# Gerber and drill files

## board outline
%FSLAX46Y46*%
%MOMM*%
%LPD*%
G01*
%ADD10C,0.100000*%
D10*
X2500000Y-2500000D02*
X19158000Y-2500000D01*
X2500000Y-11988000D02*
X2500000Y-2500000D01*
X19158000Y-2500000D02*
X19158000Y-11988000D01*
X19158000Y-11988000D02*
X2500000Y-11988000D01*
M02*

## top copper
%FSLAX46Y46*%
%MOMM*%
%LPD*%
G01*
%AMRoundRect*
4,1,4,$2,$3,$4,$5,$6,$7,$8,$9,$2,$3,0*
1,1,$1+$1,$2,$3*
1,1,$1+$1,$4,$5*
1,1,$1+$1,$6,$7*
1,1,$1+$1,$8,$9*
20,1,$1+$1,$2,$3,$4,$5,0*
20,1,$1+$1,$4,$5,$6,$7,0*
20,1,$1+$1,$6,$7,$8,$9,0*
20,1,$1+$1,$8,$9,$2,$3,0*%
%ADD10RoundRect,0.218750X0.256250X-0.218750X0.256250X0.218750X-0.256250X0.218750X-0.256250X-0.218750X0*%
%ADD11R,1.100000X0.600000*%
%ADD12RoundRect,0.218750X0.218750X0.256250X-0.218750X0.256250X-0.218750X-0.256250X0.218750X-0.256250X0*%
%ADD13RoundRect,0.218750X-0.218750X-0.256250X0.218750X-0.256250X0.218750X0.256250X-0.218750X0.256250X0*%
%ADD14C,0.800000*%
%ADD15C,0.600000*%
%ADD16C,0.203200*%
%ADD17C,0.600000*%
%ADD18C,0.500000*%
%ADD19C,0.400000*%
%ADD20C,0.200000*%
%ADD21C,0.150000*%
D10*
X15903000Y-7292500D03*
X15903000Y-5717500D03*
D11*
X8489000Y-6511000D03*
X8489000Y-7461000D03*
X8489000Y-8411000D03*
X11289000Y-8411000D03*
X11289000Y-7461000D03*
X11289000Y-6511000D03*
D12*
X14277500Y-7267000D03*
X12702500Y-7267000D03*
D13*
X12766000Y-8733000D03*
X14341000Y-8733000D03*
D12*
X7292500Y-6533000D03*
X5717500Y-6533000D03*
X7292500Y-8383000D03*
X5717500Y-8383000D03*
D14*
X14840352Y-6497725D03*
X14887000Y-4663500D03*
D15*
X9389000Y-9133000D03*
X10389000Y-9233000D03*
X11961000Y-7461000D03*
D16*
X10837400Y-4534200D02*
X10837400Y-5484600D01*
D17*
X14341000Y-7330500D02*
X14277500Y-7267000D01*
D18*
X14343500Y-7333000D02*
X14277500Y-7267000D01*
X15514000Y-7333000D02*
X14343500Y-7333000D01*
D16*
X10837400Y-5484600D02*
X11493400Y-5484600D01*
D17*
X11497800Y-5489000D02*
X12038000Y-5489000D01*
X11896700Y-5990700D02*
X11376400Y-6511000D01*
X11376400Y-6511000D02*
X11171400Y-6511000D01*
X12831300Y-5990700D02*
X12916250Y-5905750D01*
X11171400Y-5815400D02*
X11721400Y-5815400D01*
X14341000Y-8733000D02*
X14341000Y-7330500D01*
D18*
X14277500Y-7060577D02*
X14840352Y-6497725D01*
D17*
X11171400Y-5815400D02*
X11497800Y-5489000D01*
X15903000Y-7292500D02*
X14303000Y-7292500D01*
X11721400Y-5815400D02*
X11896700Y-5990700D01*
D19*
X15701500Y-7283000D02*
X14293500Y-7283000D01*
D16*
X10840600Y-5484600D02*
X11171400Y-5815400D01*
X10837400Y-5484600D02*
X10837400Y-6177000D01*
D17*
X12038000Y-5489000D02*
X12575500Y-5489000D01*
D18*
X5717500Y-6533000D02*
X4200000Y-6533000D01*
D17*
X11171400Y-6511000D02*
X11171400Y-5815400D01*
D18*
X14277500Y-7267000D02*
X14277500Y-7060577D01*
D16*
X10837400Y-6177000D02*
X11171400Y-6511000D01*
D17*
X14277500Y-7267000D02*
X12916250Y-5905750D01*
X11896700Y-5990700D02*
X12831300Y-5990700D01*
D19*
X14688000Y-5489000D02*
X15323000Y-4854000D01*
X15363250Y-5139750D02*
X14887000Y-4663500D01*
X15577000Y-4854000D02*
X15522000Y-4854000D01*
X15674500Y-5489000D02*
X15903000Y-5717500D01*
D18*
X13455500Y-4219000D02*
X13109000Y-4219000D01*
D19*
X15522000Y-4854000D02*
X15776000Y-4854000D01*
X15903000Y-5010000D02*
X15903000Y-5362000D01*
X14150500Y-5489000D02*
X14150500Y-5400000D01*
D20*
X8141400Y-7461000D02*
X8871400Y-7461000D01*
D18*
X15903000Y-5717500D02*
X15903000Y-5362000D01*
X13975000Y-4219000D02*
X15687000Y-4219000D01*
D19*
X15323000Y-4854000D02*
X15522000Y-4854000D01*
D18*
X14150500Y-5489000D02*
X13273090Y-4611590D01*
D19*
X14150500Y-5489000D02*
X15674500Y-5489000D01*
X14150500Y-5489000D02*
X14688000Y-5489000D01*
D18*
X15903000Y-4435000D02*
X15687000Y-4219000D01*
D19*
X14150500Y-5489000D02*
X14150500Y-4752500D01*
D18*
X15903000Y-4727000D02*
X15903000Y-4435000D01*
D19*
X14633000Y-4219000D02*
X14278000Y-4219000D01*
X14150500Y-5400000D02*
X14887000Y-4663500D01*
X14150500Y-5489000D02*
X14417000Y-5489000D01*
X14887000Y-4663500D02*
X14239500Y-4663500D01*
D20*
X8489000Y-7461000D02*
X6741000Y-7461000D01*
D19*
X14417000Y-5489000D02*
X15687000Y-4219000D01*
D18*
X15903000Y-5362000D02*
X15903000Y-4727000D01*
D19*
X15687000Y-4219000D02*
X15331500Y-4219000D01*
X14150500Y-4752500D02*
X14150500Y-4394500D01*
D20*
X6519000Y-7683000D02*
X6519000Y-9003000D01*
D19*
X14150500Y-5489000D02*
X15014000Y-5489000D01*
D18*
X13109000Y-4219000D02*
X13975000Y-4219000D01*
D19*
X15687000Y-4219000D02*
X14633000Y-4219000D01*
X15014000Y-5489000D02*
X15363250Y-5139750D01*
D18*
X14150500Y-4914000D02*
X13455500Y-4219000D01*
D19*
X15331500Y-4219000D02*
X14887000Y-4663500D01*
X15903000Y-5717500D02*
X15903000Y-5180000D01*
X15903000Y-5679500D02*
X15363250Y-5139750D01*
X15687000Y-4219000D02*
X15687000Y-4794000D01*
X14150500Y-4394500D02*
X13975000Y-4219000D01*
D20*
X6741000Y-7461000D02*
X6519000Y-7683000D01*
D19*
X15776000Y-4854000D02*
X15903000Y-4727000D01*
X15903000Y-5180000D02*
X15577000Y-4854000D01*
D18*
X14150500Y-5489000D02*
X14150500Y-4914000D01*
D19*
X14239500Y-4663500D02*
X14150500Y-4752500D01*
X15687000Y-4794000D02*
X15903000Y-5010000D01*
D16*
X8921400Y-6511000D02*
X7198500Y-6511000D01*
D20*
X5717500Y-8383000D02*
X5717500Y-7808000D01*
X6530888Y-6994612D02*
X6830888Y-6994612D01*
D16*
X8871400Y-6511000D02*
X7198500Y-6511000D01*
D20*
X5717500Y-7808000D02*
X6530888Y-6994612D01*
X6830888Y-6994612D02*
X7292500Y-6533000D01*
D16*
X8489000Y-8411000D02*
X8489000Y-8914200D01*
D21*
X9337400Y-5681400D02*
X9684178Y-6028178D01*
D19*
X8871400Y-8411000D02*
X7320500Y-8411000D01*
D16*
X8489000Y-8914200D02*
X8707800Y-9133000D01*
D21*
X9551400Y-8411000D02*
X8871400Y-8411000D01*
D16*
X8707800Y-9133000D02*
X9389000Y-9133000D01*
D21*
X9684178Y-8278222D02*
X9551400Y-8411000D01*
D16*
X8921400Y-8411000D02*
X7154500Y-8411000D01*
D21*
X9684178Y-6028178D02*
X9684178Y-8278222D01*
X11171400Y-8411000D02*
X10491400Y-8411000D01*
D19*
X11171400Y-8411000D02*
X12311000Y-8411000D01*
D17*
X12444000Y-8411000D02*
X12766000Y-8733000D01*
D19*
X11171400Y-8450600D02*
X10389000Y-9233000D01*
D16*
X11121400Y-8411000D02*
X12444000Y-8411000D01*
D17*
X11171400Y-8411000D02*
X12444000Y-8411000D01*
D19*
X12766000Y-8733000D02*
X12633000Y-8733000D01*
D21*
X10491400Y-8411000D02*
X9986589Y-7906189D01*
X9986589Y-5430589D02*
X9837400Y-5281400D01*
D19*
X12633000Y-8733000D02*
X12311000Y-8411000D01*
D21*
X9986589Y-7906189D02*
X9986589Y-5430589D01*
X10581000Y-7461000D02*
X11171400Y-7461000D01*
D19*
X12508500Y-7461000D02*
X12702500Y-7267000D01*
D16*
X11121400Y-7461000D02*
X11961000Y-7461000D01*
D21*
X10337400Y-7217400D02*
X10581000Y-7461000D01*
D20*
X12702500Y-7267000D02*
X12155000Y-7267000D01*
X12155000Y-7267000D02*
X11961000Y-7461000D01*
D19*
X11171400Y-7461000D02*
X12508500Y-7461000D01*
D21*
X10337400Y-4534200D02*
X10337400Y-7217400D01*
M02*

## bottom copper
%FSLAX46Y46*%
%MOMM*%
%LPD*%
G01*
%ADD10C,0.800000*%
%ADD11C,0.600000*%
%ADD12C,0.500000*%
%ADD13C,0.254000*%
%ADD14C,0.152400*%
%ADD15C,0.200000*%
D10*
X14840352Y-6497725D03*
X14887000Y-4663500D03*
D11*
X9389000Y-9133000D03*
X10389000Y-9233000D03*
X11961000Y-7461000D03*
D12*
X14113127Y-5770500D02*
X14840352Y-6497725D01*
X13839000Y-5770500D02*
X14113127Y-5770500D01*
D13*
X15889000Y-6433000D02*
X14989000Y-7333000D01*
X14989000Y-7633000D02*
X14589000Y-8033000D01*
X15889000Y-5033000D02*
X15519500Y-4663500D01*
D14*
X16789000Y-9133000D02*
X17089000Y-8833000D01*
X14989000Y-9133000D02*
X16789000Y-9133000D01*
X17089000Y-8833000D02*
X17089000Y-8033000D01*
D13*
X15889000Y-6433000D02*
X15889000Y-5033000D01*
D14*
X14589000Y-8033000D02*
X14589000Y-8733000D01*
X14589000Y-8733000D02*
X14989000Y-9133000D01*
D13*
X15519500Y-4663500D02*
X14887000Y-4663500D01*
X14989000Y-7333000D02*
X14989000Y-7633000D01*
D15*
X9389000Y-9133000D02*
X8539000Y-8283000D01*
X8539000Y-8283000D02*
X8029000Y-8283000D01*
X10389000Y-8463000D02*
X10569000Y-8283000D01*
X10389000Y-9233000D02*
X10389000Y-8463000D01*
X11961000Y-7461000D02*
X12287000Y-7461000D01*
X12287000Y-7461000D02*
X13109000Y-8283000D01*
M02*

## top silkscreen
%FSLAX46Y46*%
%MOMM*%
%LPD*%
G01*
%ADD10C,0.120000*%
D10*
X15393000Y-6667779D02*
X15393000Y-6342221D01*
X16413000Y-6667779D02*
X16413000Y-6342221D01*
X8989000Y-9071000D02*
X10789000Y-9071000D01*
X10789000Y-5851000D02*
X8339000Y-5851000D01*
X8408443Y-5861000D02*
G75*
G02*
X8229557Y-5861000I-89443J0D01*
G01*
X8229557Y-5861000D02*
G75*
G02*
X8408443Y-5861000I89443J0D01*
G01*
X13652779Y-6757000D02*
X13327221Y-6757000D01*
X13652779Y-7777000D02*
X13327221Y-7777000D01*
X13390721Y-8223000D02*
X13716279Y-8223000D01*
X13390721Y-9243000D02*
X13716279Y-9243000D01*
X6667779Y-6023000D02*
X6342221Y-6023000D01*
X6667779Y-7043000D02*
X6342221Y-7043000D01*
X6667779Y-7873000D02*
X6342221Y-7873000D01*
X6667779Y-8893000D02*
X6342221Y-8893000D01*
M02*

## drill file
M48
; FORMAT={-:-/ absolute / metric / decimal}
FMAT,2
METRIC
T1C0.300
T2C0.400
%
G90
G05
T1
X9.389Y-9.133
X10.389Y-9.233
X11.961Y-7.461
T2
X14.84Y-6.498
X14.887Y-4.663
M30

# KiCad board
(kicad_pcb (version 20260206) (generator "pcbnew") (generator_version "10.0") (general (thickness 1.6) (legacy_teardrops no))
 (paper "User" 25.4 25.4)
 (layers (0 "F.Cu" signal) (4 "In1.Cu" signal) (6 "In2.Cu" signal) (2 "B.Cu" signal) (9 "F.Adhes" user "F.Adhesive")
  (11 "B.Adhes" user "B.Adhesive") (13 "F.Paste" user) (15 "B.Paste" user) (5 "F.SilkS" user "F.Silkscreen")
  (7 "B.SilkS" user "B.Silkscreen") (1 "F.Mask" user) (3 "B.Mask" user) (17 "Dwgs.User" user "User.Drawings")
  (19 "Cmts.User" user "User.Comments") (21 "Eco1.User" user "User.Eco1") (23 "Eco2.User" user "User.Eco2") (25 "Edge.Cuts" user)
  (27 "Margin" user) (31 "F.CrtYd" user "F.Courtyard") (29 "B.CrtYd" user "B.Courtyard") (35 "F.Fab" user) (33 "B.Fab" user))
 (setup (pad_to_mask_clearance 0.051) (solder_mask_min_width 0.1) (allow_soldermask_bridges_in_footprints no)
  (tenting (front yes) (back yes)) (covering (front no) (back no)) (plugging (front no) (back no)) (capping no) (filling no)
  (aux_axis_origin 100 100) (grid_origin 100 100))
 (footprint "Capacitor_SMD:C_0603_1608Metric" (layer "F.Cu") (at 15.903 6.505 90)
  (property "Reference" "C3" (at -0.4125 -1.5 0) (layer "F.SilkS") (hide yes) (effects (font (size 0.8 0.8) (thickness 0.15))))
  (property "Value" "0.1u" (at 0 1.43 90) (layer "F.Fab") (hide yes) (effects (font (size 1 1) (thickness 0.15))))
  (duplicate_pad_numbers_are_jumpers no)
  (fp_line (start -0.162779 -0.51) (end 0.162779 -0.51) (stroke (width 0.12) (type solid)) (layer "F.SilkS"))
  (fp_line (start -0.162779 0.51) (end 0.162779 0.51) (stroke (width 0.12) (type solid)) (layer "F.SilkS"))
  (pad "1" smd roundrect (at -0.7875 0 90) (size 0.875 0.95) (layers "F.Cu" "F.Mask" "F.Paste") (roundrect_rratio 0.25) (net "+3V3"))
  (pad "2" smd roundrect (at 0.7875 0 90) (size 0.875 0.95) (layers "F.Cu" "F.Mask" "F.Paste") (roundrect_rratio 0.25) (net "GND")))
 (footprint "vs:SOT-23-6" (layer "F.Cu") (at 9.889 7.461)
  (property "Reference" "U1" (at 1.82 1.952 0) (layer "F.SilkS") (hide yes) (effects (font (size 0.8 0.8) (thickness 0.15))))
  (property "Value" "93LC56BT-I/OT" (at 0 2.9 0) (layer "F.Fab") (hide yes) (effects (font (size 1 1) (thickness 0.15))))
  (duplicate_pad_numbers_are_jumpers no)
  (fp_line (start -0.9 1.61) (end 0.9 1.61) (stroke (width 0.12) (type solid)) (layer "F.SilkS"))
  (fp_line (start 0.9 -1.61) (end -1.55 -1.61) (stroke (width 0.12) (type solid)) (layer "F.SilkS"))
  (fp_circle (center -1.57 -1.6) (end -1.53 -1.52) (stroke (width 0.12) (type solid)) (fill no) (layer "F.SilkS"))
  (pad "1" smd rect (at -1.4 -0.95) (size 1.1 0.6) (layers "F.Cu" "F.Mask" "F.Paste") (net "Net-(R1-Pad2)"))
  (pad "2" smd rect (at -1.4 0) (size 1.1 0.6) (layers "F.Cu" "F.Mask" "F.Paste") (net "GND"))
  (pad "3" smd rect (at -1.4 0.95) (size 1.1 0.6) (layers "F.Cu" "F.Mask" "F.Paste") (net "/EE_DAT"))
  (pad "4" smd rect (at 1.4 0.95) (size 1.1 0.6) (layers "F.Cu" "F.Mask" "F.Paste") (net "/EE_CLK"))
  (pad "5" smd rect (at 1.4 0) (size 1.1 0.6) (layers "F.Cu" "F.Mask" "F.Paste") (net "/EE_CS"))
  (pad "6" smd rect (at 1.4 -0.95) (size 1.1 0.6) (layers "F.Cu" "F.Mask" "F.Paste") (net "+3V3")))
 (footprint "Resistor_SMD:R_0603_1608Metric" (layer "F.Cu") (at 13.49 7.267 180)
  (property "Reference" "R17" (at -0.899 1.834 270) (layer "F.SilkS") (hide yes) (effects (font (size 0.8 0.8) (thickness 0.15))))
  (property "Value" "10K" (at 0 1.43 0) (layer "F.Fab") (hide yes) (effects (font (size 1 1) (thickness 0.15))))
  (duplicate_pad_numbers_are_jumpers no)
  (fp_line (start -0.162779 0.51) (end 0.162779 0.51) (stroke (width 0.12) (type solid)) (layer "F.SilkS"))
  (fp_line (start -0.162779 -0.51) (end 0.162779 -0.51) (stroke (width 0.12) (type solid)) (layer "F.SilkS"))
  (pad "1" smd roundrect (at -0.7875 0 180) (size 0.875 0.95) (layers "F.Cu" "F.Mask" "F.Paste") (roundrect_rratio 0.25) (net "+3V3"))
  (pad "2" smd roundrect (at 0.7875 0 180) (size 0.875 0.95) (layers "F.Cu" "F.Mask" "F.Paste") (roundrect_rratio 0.25) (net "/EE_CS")))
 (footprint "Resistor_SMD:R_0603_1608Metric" (layer "F.Cu") (at 13.5535 8.733)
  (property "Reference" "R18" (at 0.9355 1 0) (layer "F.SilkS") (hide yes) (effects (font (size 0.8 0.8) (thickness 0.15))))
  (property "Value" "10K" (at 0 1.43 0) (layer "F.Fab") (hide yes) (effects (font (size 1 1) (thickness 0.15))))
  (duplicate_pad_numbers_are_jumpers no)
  (fp_line (start -0.162779 -0.51) (end 0.162779 -0.51) (stroke (width 0.12) (type solid)) (layer "F.SilkS"))
  (fp_line (start -0.162779 0.51) (end 0.162779 0.51) (stroke (width 0.12) (type solid)) (layer "F.SilkS"))
  (pad "1" smd roundrect (at -0.7875 0) (size 0.875 0.95) (layers "F.Cu" "F.Mask" "F.Paste") (roundrect_rratio 0.25) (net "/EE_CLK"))
  (pad "2" smd roundrect (at 0.7875 0) (size 0.875 0.95) (layers "F.Cu" "F.Mask" "F.Paste") (roundrect_rratio 0.25) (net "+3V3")))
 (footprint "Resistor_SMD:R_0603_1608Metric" (layer "F.Cu") (at 6.505 6.533 180)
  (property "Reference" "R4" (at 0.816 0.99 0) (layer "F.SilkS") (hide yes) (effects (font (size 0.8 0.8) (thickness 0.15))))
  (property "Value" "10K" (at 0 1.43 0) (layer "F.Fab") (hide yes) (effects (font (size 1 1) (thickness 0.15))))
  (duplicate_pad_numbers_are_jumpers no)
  (fp_line (start -0.162779 0.51) (end 0.162779 0.51) (stroke (width 0.12) (type solid)) (layer "F.SilkS"))
  (fp_line (start -0.162779 -0.51) (end 0.162779 -0.51) (stroke (width 0.12) (type solid)) (layer "F.SilkS"))
  (pad "1" smd roundrect (at -0.7875 0 180) (size 0.875 0.95) (layers "F.Cu" "F.Mask" "F.Paste") (roundrect_rratio 0.25)
   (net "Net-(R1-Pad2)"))
  (pad "2" smd roundrect (at 0.7875 0 180) (size 0.875 0.95) (layers "F.Cu" "F.Mask" "F.Paste") (roundrect_rratio 0.25) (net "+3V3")))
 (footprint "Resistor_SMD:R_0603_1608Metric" (layer "F.Cu") (at 6.505 8.383 180)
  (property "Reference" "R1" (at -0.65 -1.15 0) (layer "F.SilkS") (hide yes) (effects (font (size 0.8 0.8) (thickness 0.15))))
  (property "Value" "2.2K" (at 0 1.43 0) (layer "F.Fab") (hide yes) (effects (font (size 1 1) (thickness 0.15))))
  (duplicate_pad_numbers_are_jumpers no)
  (fp_line (start -0.162779 0.51) (end 0.162779 0.51) (stroke (width 0.12) (type solid)) (layer "F.SilkS"))
  (fp_line (start -0.162779 -0.51) (end 0.162779 -0.51) (stroke (width 0.12) (type solid)) (layer "F.SilkS"))
  (pad "1" smd roundrect (at -0.7875 0 180) (size 0.875 0.95) (layers "F.Cu" "F.Mask" "F.Paste") (roundrect_rratio 0.25) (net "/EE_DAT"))
  (pad "2" smd roundrect (at 0.7875 0 180) (size 0.875 0.95) (layers "F.Cu" "F.Mask" "F.Paste") (roundrect_rratio 0.25)
   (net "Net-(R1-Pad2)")))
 (gr_line (start 2.5 2.5) (end 19.158 2.5) (stroke (width 0.1) (type default)) (layer "Edge.Cuts"))
 (gr_line (start 2.5 11.988) (end 2.5 2.5) (stroke (width 0.1) (type default)) (layer "Edge.Cuts"))
 (gr_line (start 19.158 2.5) (end 19.158 11.988) (stroke (width 0.1) (type default)) (layer "Edge.Cuts"))
 (gr_line (start 19.158 11.988) (end 2.5 11.988) (stroke (width 0.1) (type default)) (layer "Edge.Cuts"))
 (segment (start 10.8374 4.5342) (end 10.8374 5.4846) (width 0.2032) (layer "F.Cu") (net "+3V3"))
 (segment (start 14.341 7.3305) (end 14.2775 7.267) (width 0.6) (layer "F.Cu") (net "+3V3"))
 (segment (start 14.3435 7.333) (end 14.2775 7.267) (width 0.5) (layer "F.Cu") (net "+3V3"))
 (segment (start 15.514 7.333) (end 14.3435 7.333) (width 0.5) (layer "F.Cu") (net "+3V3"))
 (segment (start 10.8374 5.4846) (end 11.4934 5.4846) (width 0.2032) (layer "F.Cu") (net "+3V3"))
 (segment (start 11.4978 5.489) (end 12.038 5.489) (width 0.6) (layer "F.Cu") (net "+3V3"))
 (segment (start 11.8967 5.9907) (end 11.3764 6.511) (width 0.6) (layer "F.Cu") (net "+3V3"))
 (segment (start 11.3764 6.511) (end 11.1714 6.511) (width 0.6) (layer "F.Cu") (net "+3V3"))
 (segment (start 12.8313 5.9907) (end 12.91625 5.90575) (width 0.6) (layer "F.Cu") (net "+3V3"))
 (segment (start 11.1714 5.8154) (end 11.7214 5.8154) (width 0.6) (layer "F.Cu") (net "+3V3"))
 (segment (start 14.341 8.733) (end 14.341 7.3305) (width 0.6) (layer "F.Cu") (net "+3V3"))
 (segment (start 14.2775 7.060577) (end 14.840352 6.497725) (width 0.5) (layer "F.Cu") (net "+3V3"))
 (segment (start 11.1714 5.8154) (end 11.4978 5.489) (width 0.6) (layer "F.Cu") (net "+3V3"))
 (segment (start 15.903 7.2925) (end 14.303 7.2925) (width 0.6) (layer "F.Cu") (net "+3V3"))
 (segment (start 11.7214 5.8154) (end 11.8967 5.9907) (width 0.6) (layer "F.Cu") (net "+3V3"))
 (segment (start 15.7015 7.283) (end 14.2935 7.283) (width 0.4) (layer "F.Cu") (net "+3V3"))
 (segment (start 10.8406 5.4846) (end 11.1714 5.8154) (width 0.2032) (layer "F.Cu") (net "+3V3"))
 (segment (start 10.8374 5.4846) (end 10.8374 6.177) (width 0.2032) (layer "F.Cu") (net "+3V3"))
 (segment (start 12.038 5.489) (end 12.5755 5.489) (width 0.6) (layer "F.Cu") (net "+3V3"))
 (segment (start 5.7175 6.533) (end 4.2 6.533) (width 0.5) (layer "F.Cu") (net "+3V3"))
 (segment (start 11.1714 6.511) (end 11.1714 5.8154) (width 0.6) (layer "F.Cu") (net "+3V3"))
 (segment (start 14.2775 7.267) (end 14.2775 7.060577) (width 0.5) (layer "F.Cu") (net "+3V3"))
 (segment (start 10.8374 6.177) (end 11.1714 6.511) (width 0.2032) (layer "F.Cu") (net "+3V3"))
 (segment (start 14.2775 7.267) (end 12.91625 5.90575) (width 0.6) (layer "F.Cu") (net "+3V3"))
 (segment (start 11.8967 5.9907) (end 12.8313 5.9907) (width 0.6) (layer "F.Cu") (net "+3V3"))
 (via (at 14.840352 6.497725) (size 0.8) (drill 0.4) (layers "F.Cu" "B.Cu") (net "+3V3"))
 (segment (start 14.113127 5.7705) (end 14.840352 6.497725) (width 0.5) (layer "B.Cu") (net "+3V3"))
 (segment (start 13.839 5.7705) (end 14.113127 5.7705) (width 0.5) (layer "B.Cu") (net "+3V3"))
 (segment (start 14.688 5.489) (end 15.323 4.854) (width 0.4) (layer "F.Cu") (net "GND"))
 (segment (start 15.36325 5.13975) (end 14.887 4.6635) (width 0.4) (layer "F.Cu") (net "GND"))
 (segment (start 15.577 4.854) (end 15.522 4.854) (width 0.4) (layer "F.Cu") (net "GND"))
 (segment (start 15.6745 5.489) (end 15.903 5.7175) (width 0.4) (layer "F.Cu") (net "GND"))
 (segment (start 13.4555 4.219) (end 13.109 4.219) (width 0.5) (layer "F.Cu") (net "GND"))
 (segment (start 15.522 4.854) (end 15.776 4.854) (width 0.4) (layer "F.Cu") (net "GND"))
 (segment (start 15.903 5.01) (end 15.903 5.362) (width 0.4) (layer "F.Cu") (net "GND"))
 (segment (start 14.1505 5.489) (end 14.1505 5.4) (width 0.4) (layer "F.Cu") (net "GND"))
 (segment (start 8.1414 7.461) (end 8.8714 7.461) (width 0.2) (layer "F.Cu") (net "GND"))
 (segment (start 15.903 5.7175) (end 15.903 5.362) (width 0.5) (layer "F.Cu") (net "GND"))
 (segment (start 13.975 4.219) (end 15.687 4.219) (width 0.5) (layer "F.Cu") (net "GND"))
 (segment (start 15.323 4.854) (end 15.522 4.854) (width 0.4) (layer "F.Cu") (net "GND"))
 (segment (start 14.1505 5.489) (end 13.27309 4.61159) (width 0.5) (layer "F.Cu") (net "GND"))
 (segment (start 14.1505 5.489) (end 15.6745 5.489) (width 0.4) (layer "F.Cu") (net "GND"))
 (segment (start 14.1505 5.489) (end 14.688 5.489) (width 0.4) (layer "F.Cu") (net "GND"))
 (segment (start 15.903 4.435) (end 15.687 4.219) (width 0.5) (layer "F.Cu") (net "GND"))
 (segment (start 14.1505 5.489) (end 14.1505 4.7525) (width 0.4) (layer "F.Cu") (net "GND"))
 (segment (start 15.903 4.727) (end 15.903 4.435) (width 0.5) (layer "F.Cu") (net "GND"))
 (segment (start 14.633 4.219) (end 14.278 4.219) (width 0.4) (layer "F.Cu") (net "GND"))
 (segment (start 14.1505 5.4) (end 14.887 4.6635) (width 0.4) (layer "F.Cu") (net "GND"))
 (segment (start 14.1505 5.489) (end 14.417 5.489) (width 0.4) (layer "F.Cu") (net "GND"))
 (segment (start 14.887 4.6635) (end 14.2395 4.6635) (width 0.4) (layer "F.Cu") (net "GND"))
 (segment (start 8.489 7.461) (end 6.741 7.461) (width 0.2) (layer "F.Cu") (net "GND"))
 (segment (start 14.417 5.489) (end 15.687 4.219) (width 0.4) (layer "F.Cu") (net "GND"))
 (segment (start 15.903 5.362) (end 15.903 4.727) (width 0.5) (layer "F.Cu") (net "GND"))
 (segment (start 15.687 4.219) (end 15.3315 4.219) (width 0.4) (layer "F.Cu") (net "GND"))
 (segment (start 14.1505 4.7525) (end 14.1505 4.3945) (width 0.4) (layer "F.Cu") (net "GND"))
 (segment (start 6.519 7.683) (end 6.519 9.003) (width 0.2) (layer "F.Cu") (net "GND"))
 (segment (start 14.1505 5.489) (end 15.014 5.489) (width 0.4) (layer "F.Cu") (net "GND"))
 (segment (start 13.109 4.219) (end 13.975 4.219) (width 0.5) (layer "F.Cu") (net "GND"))
 (segment (start 15.687 4.219) (end 14.633 4.219) (width 0.4) (layer "F.Cu") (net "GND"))
 (segment (start 15.014 5.489) (end 15.36325 5.13975) (width 0.4) (layer "F.Cu") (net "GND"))
 (segment (start 14.1505 4.914) (end 13.4555 4.219) (width 0.5) (layer "F.Cu") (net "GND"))
 (segment (start 15.3315 4.219) (end 14.887 4.6635) (width 0.4) (layer "F.Cu") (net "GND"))
 (segment (start 15.903 5.7175) (end 15.903 5.18) (width 0.4) (layer "F.Cu") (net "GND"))
 (segment (start 15.903 5.6795) (end 15.36325 5.13975) (width 0.4) (layer "F.Cu") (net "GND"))
 (segment (start 15.687 4.219) (end 15.687 4.794) (width 0.4) (layer "F.Cu") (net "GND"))
 (segment (start 14.1505 4.3945) (end 13.975 4.219) (width 0.4) (layer "F.Cu") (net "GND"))
 (segment (start 6.741 7.461) (end 6.519 7.683) (width 0.2) (layer "F.Cu") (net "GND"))
 (segment (start 15.776 4.854) (end 15.903 4.727) (width 0.4) (layer "F.Cu") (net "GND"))
 (segment (start 15.903 5.18) (end 15.577 4.854) (width 0.4) (layer "F.Cu") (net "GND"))
 (segment (start 14.1505 5.489) (end 14.1505 4.914) (width 0.5) (layer "F.Cu") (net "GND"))
 (segment (start 14.2395 4.6635) (end 14.1505 4.7525) (width 0.4) (layer "F.Cu") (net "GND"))
 (segment (start 15.687 4.794) (end 15.903 5.01) (width 0.4) (layer "F.Cu") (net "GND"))
 (via (at 14.887 4.6635) (size 0.8) (drill 0.4) (layers "F.Cu" "B.Cu") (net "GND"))
 (segment (start 15.889 6.433) (end 14.989 7.333) (width 0.254) (layer "B.Cu") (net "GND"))
 (segment (start 14.989 7.633) (end 14.589 8.033) (width 0.254) (layer "B.Cu") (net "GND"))
 (segment (start 15.889 5.033) (end 15.5195 4.6635) (width 0.254) (layer "B.Cu") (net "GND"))
 (segment (start 16.789 9.133) (end 17.089 8.833) (width 0.1524) (layer "B.Cu") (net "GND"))
 (segment (start 14.989 9.133) (end 16.789 9.133) (width 0.1524) (layer "B.Cu") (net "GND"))
 (segment (start 17.089 8.833) (end 17.089 8.033) (width 0.1524) (layer "B.Cu") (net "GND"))
 (segment (start 15.889 6.433) (end 15.889 5.033) (width 0.254) (layer "B.Cu") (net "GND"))
 (segment (start 14.589 8.033) (end 14.589 8.733) (width 0.1524) (layer "B.Cu") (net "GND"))
 (segment (start 14.589 8.733) (end 14.989 9.133) (width 0.1524) (layer "B.Cu") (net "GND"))
 (segment (start 15.5195 4.6635) (end 14.887 4.6635) (width 0.254) (layer "B.Cu") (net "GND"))
 (segment (start 14.989 7.333) (end 14.989 7.633) (width 0.254) (layer "B.Cu") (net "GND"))
 (segment (start 8.9214 6.511) (end 7.1985 6.511) (width 0.2032) (layer "F.Cu") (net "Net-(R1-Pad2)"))
 (segment (start 5.7175 8.383) (end 5.7175 7.808) (width 0.2) (layer "F.Cu") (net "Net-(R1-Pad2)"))
 (segment (start 6.530888 6.994612) (end 6.830888 6.994612) (width 0.2) (layer "F.Cu") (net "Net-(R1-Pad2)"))
 (segment (start 8.8714 6.511) (end 7.1985 6.511) (width 0.2032) (layer "F.Cu") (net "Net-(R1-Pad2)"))
 (segment (start 5.7175 7.808) (end 6.530888 6.994612) (width 0.2) (layer "F.Cu") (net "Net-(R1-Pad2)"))
 (segment (start 6.830888 6.994612) (end 7.2925 6.533) (width 0.2) (layer "F.Cu") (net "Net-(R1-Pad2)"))
 (segment (start 8.489 8.411) (end 8.489 8.9142) (width 0.2032) (layer "F.Cu") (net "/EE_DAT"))
 (segment (start 9.3374 5.6814) (end 9.684178 6.028178) (width 0.15) (layer "F.Cu") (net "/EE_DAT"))
 (segment (start 8.8714 8.411) (end 7.3205 8.411) (width 0.4) (layer "F.Cu") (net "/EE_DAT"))
 (segment (start 8.489 8.9142) (end 8.7078 9.133) (width 0.2032) (layer "F.Cu") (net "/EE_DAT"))
 (segment (start 9.5514 8.411) (end 8.8714 8.411) (width 0.15) (layer "F.Cu") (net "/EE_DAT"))
 (segment (start 8.7078 9.133) (end 9.389 9.133) (width 0.2032) (layer "F.Cu") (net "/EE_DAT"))
 (segment (start 9.684178 8.278222) (end 9.5514 8.411) (width 0.15) (layer "F.Cu") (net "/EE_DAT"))
 (segment (start 8.9214 8.411) (end 7.1545 8.411) (width 0.2032) (layer "F.Cu") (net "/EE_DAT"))
 (segment (start 9.684178 6.028178) (end 9.684178 8.278222) (width 0.15) (layer "F.Cu") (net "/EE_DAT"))
 (via (at 9.389 9.133) (size 0.6) (drill 0.3) (layers "F.Cu" "B.Cu") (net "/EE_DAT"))
 (segment (start 9.389 9.133) (end 8.539 8.283) (width 0.2) (layer "B.Cu") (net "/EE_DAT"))
 (segment (start 8.539 8.283) (end 8.029 8.283) (width 0.2) (layer "B.Cu") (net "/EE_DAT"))
 (segment (start 11.1714 8.411) (end 10.4914 8.411) (width 0.15) (layer "F.Cu") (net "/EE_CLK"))
 (segment (start 11.1714 8.411) (end 12.311 8.411) (width 0.4) (layer "F.Cu") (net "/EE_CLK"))
 (segment (start 12.444 8.411) (end 12.766 8.733) (width 0.6) (layer "F.Cu") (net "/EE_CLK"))
 (segment (start 11.1714 8.4506) (end 10.389 9.233) (width 0.4) (layer "F.Cu") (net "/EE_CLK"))
 (segment (start 11.1214 8.411) (end 12.444 8.411) (width 0.2032) (layer "F.Cu") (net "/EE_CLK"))
 (segment (start 11.1714 8.411) (end 12.444 8.411) (width 0.6) (layer "F.Cu") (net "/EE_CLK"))
 (segment (start 12.766 8.733) (end 12.633 8.733) (width 0.4) (layer "F.Cu") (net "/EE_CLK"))
 (segment (start 10.4914 8.411) (end 9.986589 7.906189) (width 0.15) (layer "F.Cu") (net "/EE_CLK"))
 (segment (start 9.986589 5.430589) (end 9.8374 5.2814) (width 0.15) (layer "F.Cu") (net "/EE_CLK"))
 (segment (start 12.633 8.733) (end 12.311 8.411) (width 0.4) (layer "F.Cu") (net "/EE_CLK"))
 (segment (start 9.986589 7.906189) (end 9.986589 5.430589) (width 0.15) (layer "F.Cu") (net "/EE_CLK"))
 (via (at 10.389 9.233) (size 0.6) (drill 0.3) (layers "F.Cu" "B.Cu") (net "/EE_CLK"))
 (segment (start 10.389 8.463) (end 10.569 8.283) (width 0.2) (layer "B.Cu") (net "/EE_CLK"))
 (segment (start 10.389 9.233) (end 10.389 8.463) (width 0.2) (layer "B.Cu") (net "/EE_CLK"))
 (segment (start 10.581 7.461) (end 11.1714 7.461) (width 0.15) (layer "F.Cu") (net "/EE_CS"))
 (segment (start 12.5085 7.461) (end 12.7025 7.267) (width 0.4) (layer "F.Cu") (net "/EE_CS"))
 (segment (start 11.1214 7.461) (end 11.961 7.461) (width 0.2032) (layer "F.Cu") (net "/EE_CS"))
 (segment (start 10.3374 7.2174) (end 10.581 7.461) (width 0.15) (layer "F.Cu") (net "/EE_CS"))
 (segment (start 12.7025 7.267) (end 12.155 7.267) (width 0.2) (layer "F.Cu") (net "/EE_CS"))
 (segment (start 12.155 7.267) (end 11.961 7.461) (width 0.2) (layer "F.Cu") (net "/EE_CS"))
 (segment (start 11.1714 7.461) (end 12.5085 7.461) (width 0.4) (layer "F.Cu") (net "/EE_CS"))
 (segment (start 10.3374 4.5342) (end 10.3374 7.2174) (width 0.15) (layer "F.Cu") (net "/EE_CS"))
 (via (at 11.961 7.461) (size 0.6) (drill 0.3) (layers "F.Cu" "B.Cu") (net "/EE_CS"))
 (segment (start 11.961 7.461) (end 12.287 7.461) (width 0.2) (layer "B.Cu") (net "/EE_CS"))
 (segment (start 12.287 7.461) (end 13.109 8.283) (width 0.2) (layer "B.Cu") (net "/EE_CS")))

